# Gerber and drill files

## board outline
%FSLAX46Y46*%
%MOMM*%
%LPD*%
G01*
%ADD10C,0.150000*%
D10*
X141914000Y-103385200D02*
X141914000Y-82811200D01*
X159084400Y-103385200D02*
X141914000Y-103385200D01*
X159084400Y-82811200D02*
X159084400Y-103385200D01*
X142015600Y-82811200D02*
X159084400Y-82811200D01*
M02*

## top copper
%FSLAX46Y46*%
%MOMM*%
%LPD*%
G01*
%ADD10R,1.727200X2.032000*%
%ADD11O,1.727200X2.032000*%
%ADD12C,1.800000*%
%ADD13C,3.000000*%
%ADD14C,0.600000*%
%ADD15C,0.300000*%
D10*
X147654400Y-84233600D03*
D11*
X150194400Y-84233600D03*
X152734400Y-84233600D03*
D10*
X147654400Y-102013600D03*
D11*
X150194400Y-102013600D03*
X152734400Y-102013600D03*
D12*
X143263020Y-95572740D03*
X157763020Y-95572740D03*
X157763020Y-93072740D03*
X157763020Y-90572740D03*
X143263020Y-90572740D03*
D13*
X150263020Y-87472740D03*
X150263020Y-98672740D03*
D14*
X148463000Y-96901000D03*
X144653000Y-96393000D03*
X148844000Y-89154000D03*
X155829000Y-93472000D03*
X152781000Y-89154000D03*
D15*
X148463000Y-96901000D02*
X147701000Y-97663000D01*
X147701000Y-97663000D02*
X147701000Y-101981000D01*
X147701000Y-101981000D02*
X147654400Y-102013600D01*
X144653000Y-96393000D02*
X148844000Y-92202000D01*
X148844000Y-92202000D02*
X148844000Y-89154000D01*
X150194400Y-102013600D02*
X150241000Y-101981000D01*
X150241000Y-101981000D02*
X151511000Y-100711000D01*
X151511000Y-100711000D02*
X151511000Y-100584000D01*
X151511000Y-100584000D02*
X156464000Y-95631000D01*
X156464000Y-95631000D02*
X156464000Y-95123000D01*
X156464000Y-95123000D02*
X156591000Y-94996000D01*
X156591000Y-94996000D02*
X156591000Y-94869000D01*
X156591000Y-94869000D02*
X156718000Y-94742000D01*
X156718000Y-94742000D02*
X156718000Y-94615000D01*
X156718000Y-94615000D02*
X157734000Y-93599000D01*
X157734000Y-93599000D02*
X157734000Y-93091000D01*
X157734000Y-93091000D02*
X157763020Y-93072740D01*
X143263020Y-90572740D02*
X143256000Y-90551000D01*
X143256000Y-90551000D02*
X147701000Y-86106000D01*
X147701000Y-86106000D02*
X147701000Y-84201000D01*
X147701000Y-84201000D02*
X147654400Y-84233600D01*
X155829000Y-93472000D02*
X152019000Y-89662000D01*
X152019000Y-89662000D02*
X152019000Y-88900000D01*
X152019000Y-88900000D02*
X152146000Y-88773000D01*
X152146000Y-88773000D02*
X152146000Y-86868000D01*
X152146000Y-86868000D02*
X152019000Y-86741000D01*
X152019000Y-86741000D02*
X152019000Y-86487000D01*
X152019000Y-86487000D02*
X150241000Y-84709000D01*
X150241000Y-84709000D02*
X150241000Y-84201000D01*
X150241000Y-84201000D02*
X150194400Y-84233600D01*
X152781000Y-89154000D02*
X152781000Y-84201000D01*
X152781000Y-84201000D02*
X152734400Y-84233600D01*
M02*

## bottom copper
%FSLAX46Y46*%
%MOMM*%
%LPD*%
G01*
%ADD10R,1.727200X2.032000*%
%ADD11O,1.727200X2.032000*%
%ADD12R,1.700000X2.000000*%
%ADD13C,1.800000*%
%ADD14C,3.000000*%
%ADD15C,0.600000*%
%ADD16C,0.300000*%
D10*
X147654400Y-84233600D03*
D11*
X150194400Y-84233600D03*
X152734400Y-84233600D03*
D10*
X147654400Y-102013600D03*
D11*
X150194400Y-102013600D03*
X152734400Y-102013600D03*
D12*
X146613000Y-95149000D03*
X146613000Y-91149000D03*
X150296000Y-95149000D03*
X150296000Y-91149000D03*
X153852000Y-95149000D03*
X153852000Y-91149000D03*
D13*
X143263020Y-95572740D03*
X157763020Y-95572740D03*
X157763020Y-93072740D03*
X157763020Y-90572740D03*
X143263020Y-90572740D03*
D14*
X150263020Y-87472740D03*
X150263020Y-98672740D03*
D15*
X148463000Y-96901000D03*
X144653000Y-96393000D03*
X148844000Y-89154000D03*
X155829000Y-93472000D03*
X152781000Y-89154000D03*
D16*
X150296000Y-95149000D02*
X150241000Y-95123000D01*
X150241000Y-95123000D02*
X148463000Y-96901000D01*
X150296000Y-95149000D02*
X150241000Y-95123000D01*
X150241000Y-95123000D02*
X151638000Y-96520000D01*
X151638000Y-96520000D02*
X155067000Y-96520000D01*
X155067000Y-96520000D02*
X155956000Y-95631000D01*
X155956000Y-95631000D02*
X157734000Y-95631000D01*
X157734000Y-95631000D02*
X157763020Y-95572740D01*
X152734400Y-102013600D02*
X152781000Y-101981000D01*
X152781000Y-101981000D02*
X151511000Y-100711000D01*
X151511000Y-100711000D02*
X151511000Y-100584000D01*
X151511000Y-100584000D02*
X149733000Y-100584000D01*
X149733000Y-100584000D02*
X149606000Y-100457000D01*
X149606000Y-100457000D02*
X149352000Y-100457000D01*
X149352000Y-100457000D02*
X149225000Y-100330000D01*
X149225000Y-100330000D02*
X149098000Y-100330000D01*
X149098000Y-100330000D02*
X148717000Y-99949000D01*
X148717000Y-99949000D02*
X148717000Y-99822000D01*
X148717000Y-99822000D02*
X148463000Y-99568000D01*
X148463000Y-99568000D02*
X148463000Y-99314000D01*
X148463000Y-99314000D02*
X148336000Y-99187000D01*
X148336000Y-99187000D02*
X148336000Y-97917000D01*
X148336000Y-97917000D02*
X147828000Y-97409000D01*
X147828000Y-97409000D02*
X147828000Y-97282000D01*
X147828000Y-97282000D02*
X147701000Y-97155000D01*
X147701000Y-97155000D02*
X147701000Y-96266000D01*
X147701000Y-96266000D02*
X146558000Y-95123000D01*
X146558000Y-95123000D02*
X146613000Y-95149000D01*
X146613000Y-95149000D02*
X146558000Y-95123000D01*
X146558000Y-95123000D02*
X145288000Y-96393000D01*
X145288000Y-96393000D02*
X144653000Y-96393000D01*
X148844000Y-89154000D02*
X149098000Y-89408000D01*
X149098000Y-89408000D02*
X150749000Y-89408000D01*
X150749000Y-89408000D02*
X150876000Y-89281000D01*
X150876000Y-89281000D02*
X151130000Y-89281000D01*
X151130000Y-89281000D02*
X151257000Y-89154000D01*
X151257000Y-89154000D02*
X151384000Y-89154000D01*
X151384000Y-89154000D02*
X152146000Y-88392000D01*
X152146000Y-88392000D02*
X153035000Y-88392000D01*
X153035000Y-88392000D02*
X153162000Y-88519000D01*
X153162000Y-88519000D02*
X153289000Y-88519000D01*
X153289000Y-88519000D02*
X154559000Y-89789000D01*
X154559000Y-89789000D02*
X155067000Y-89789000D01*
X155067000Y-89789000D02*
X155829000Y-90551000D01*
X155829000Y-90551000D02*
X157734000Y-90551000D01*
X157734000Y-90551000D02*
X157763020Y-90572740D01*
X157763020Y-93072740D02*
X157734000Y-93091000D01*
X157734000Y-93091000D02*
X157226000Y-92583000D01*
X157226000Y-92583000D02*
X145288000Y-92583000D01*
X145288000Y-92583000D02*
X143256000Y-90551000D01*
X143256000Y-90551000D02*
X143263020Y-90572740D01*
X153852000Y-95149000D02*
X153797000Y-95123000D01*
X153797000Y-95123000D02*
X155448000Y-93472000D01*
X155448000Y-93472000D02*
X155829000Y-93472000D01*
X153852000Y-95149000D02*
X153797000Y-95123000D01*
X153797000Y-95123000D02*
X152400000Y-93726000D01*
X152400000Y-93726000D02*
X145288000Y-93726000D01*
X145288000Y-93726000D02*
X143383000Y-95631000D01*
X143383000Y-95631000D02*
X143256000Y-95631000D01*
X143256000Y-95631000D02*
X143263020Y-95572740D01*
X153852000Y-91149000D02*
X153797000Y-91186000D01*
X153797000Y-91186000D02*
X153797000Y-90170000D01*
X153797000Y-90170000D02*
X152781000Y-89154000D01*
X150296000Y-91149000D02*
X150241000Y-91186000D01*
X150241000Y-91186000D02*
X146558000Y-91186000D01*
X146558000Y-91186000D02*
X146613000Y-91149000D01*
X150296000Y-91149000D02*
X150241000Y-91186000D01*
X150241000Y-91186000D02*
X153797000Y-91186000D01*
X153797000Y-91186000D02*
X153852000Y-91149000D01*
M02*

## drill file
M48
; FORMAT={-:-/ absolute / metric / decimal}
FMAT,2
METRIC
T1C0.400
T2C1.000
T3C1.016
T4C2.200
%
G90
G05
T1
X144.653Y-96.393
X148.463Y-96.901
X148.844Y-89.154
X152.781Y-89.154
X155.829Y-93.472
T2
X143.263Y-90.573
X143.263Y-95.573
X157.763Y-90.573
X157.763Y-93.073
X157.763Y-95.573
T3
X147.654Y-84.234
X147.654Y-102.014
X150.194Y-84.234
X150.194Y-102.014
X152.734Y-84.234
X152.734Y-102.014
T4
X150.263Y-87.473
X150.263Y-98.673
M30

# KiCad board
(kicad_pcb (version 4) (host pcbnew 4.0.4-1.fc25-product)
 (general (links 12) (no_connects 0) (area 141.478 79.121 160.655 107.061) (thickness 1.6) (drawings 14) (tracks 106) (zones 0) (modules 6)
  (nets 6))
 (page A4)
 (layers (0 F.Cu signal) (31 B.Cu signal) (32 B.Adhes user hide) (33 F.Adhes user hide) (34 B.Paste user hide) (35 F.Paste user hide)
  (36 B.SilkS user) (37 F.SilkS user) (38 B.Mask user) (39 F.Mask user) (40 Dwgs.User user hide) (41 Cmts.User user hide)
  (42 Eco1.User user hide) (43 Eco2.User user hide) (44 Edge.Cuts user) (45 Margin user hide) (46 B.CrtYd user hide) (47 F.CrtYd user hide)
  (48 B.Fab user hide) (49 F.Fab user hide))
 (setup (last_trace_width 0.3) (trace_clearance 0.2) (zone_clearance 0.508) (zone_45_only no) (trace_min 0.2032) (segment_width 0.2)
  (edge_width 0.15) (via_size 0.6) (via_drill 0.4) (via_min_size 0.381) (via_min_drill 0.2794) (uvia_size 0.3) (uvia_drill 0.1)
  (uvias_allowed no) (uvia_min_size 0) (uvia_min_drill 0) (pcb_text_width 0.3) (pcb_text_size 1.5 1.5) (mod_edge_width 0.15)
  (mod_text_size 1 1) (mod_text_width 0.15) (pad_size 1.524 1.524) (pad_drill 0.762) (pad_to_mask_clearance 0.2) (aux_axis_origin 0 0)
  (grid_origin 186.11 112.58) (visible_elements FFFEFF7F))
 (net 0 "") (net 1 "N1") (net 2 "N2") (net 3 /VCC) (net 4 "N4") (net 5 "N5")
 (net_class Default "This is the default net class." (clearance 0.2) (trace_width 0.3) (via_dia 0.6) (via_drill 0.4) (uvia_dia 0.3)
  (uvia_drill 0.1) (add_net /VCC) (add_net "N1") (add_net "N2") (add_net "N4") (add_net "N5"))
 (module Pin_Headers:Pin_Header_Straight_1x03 (layer F.Cu) (at 147.6544 84.2336 90)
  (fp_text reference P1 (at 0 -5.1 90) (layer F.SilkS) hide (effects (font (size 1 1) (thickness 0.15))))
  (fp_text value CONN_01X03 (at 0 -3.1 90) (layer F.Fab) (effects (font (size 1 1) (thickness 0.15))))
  (pad 1 thru_hole rect (at 0 0 90) (size 2.032 1.7272) (drill 1.016) (layers *.Cu *.Mask F.SilkS) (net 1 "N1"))
  (pad 2 thru_hole oval (at 0 2.54 90) (size 2.032 1.7272) (drill 1.016) (layers *.Cu *.Mask F.SilkS) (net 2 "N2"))
  (pad 3 thru_hole oval (at 0 5.08 90) (size 2.032 1.7272) (drill 1.016) (layers *.Cu *.Mask F.SilkS) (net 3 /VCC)))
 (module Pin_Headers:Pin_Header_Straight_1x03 (layer F.Cu) (at 147.6544 102.0136 90)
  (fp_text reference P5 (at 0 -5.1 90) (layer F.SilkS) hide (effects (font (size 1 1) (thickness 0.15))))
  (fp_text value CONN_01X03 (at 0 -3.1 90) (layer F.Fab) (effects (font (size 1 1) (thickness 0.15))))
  (pad 1 thru_hole rect (at 0 0 90) (size 2.032 1.7272) (drill 1.016) (layers *.Cu *.Mask F.SilkS) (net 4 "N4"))
  (pad 2 thru_hole oval (at 0 2.54 90) (size 2.032 1.7272) (drill 1.016) (layers *.Cu *.Mask F.SilkS) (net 1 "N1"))
  (pad 3 thru_hole oval (at 0 5.08 90) (size 2.032 1.7272) (drill 1.016) (layers *.Cu *.Mask F.SilkS) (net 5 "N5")))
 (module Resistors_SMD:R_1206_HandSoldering (layer B.Cu) (at 146.613 93.149 90)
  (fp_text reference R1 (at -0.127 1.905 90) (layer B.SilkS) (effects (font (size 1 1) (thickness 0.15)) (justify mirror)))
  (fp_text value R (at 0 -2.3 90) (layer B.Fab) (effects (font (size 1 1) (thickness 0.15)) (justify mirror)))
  (pad 1 smd rect (at -2 0 90) (size 2 1.7) (layers B.Cu B.Paste B.Mask) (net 5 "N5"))
  (pad 2 smd rect (at 2 0 90) (size 2 1.7) (layers B.Cu B.Paste B.Mask) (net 3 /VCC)))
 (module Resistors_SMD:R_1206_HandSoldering (layer B.Cu) (at 150.296 93.149 90)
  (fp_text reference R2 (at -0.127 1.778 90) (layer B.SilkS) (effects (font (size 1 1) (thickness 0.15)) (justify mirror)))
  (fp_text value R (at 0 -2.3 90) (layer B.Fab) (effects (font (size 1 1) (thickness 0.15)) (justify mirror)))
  (pad 1 smd rect (at -2 0 90) (size 2 1.7) (layers B.Cu B.Paste B.Mask) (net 4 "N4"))
  (pad 2 smd rect (at 2 0 90) (size 2 1.7) (layers B.Cu B.Paste B.Mask) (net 3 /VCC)))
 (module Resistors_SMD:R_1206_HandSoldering (layer B.Cu) (at 153.852 93.149 90)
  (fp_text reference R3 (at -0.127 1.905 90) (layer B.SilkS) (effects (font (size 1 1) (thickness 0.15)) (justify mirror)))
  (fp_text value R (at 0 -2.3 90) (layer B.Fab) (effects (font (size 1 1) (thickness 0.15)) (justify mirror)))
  (pad 1 smd rect (at -2 0 90) (size 2 1.7) (layers B.Cu B.Paste B.Mask) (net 2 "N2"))
  (pad 2 smd rect (at 2 0 90) (size 2 1.7) (layers B.Cu B.Paste B.Mask) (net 3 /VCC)))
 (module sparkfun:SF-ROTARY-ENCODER (layer F.Cu) (at 150.26302 93.07274 90)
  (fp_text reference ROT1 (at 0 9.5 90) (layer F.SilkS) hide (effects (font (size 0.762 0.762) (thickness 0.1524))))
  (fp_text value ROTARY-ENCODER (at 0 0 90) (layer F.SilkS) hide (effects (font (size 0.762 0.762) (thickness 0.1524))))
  (pad 1 thru_hole circle (at -2.5 -7 90) (size 1.8 1.8) (drill 1) (layers *.Cu *.Mask F.SilkS) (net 2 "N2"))
  (pad 2 thru_hole circle (at -2.5 7.5 90) (size 1.8 1.8) (drill 1) (layers *.Cu *.Mask F.SilkS) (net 4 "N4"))
  (pad 3 thru_hole circle (at 0 7.5 90) (size 1.8 1.8) (drill 1) (layers *.Cu *.Mask F.SilkS) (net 1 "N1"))
  (pad 4 thru_hole circle (at 2.5 7.5 90) (size 1.8 1.8) (drill 1) (layers *.Cu *.Mask F.SilkS) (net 5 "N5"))
  (pad 5 thru_hole circle (at 2.5 -7 90) (size 1.8 1.8) (drill 1) (layers *.Cu *.Mask F.SilkS) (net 1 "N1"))
  (pad "" thru_hole circle (at 5.6 0 90) (size 3 3) (drill 2.2) (layers *.Cu *.Mask F.SilkS))
  (pad "" thru_hole circle (at -5.6 0 90) (size 3 3) (drill 2.2) (layers *.Cu *.Mask F.SilkS)))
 (gr_line (start 141.914 103.3852) (end 141.914 82.8112) (angle 90) (layer Edge.Cuts) (width 0.15))
 (gr_line (start 159.0844 103.3852) (end 141.914 103.3852) (angle 90) (layer Edge.Cuts) (width 0.15))
 (gr_line (start 159.0844 82.8112) (end 159.0844 103.3852) (angle 90) (layer Edge.Cuts) (width 0.15))
 (gr_line (start 142.0156 82.8112) (end 159.0844 82.8112) (angle 90) (layer Edge.Cuts) (width 0.15))
 (segment (start 150.296 95.149) (end 150.241 95.123) (width 0.3) (layer B.Cu) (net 4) (status 80000))
 (segment (start 150.241 95.123) (end 148.463 96.901) (width 0.3) (layer B.Cu) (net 4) (status 80000))
 (via (at 148.463 96.901) (size 0.6) (layers F.Cu B.Cu) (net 4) (status 80000))
 (segment (start 148.463 96.901) (end 147.701 97.663) (width 0.3) (layer F.Cu) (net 4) (status 80000))
 (segment (start 147.701 97.663) (end 147.701 101.981) (width 0.3) (layer F.Cu) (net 4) (status 80000))
 (segment (start 147.701 101.981) (end 147.6544 102.0136) (width 0.3) (layer F.Cu) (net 4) (status 80000))
 (segment (start 150.296 95.149) (end 150.241 95.123) (width 0.3) (layer B.Cu) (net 4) (status 80000))
 (segment (start 150.241 95.123) (end 151.638 96.52) (width 0.3) (layer B.Cu) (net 4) (status 80000))
 (segment (start 151.638 96.52) (end 155.067 96.52) (width 0.3) (layer B.Cu) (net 4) (status 80000))
 (segment (start 155.067 96.52) (end 155.956 95.631) (width 0.3) (layer B.Cu) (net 4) (status 80000))
 (segment (start 155.956 95.631) (end 157.734 95.631) (width 0.3) (layer B.Cu) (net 4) (status 80000))
 (segment (start 157.734 95.631) (end 157.76302 95.57274) (width 0.3) (layer B.Cu) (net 4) (status 80000))
 (segment (start 152.7344 102.0136) (end 152.781 101.981) (width 0.3) (layer B.Cu) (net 5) (status 80000))
 (segment (start 152.781 101.981) (end 151.511 100.711) (width 0.3) (layer B.Cu) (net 5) (status 80000))
 (segment (start 151.511 100.711) (end 151.511 100.584) (width 0.3) (layer B.Cu) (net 5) (status 80000))
 (segment (start 151.511 100.584) (end 149.733 100.584) (width 0.3) (layer B.Cu) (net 5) (status 80000))
 (segment (start 149.733 100.584) (end 149.606 100.457) (width 0.3) (layer B.Cu) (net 5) (status 80000))
 (segment (start 149.606 100.457) (end 149.352 100.457) (width 0.3) (layer B.Cu) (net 5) (status 80000))
 (segment (start 149.352 100.457) (end 149.225 100.33) (width 0.3) (layer B.Cu) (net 5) (status 80000))
 (segment (start 149.225 100.33) (end 149.098 100.33) (width 0.3) (layer B.Cu) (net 5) (status 80000))
 (segment (start 149.098 100.33) (end 148.717 99.949) (width 0.3) (layer B.Cu) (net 5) (status 80000))
 (segment (start 148.717 99.949) (end 148.717 99.822) (width 0.3) (layer B.Cu) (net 5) (status 80000))
 (segment (start 148.717 99.822) (end 148.463 99.568) (width 0.3) (layer B.Cu) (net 5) (status 80000))
 (segment (start 148.463 99.568) (end 148.463 99.314) (width 0.3) (layer B.Cu) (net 5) (status 80000))
 (segment (start 148.463 99.314) (end 148.336 99.187) (width 0.3) (layer B.Cu) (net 5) (status 80000))
 (segment (start 148.336 99.187) (end 148.336 97.917) (width 0.3) (layer B.Cu) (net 5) (status 80000))
 (segment (start 148.336 97.917) (end 147.828 97.409) (width 0.3) (layer B.Cu) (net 5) (status 80000))
 (segment (start 147.828 97.409) (end 147.828 97.282) (width 0.3) (layer B.Cu) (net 5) (status 80000))
 (segment (start 147.828 97.282) (end 147.701 97.155) (width 0.3) (layer B.Cu) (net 5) (status 80000))
 (segment (start 147.701 97.155) (end 147.701 96.266) (width 0.3) (layer B.Cu) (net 5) (status 80000))
 (segment (start 147.701 96.266) (end 146.558 95.123) (width 0.3) (layer B.Cu) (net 5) (status 80000))
 (segment (start 146.558 95.123) (end 146.613 95.149) (width 0.3) (layer B.Cu) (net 5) (status 80000))
 (segment (start 146.613 95.149) (end 146.558 95.123) (width 0.3) (layer B.Cu) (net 5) (status 80000))
 (segment (start 146.558 95.123) (end 145.288 96.393) (width 0.3) (layer B.Cu) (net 5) (status 80000))
 (segment (start 145.288 96.393) (end 144.653 96.393) (width 0.3) (layer B.Cu) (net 5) (status 80000))
 (via (at 144.653 96.393) (size 0.6) (layers F.Cu B.Cu) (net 5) (status 80000))
 (segment (start 144.653 96.393) (end 148.844 92.202) (width 0.3) (layer F.Cu) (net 5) (status 80000))
 (segment (start 148.844 92.202) (end 148.844 89.154) (width 0.3) (layer F.Cu) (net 5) (status 80000))
 (via (at 148.844 89.154) (size 0.6) (layers F.Cu B.Cu) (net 5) (status 80000))
 (segment (start 148.844 89.154) (end 149.098 89.408) (width 0.3) (layer B.Cu) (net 5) (status 80000))
 (segment (start 149.098 89.408) (end 150.749 89.408) (width 0.3) (layer B.Cu) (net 5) (status 80000))
 (segment (start 150.749 89.408) (end 150.876 89.281) (width 0.3) (layer B.Cu) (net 5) (status 80000))
 (segment (start 150.876 89.281) (end 151.13 89.281) (width 0.3) (layer B.Cu) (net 5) (status 80000))
 (segment (start 151.13 89.281) (end 151.257 89.154) (width 0.3) (layer B.Cu) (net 5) (status 80000))
 (segment (start 151.257 89.154) (end 151.384 89.154) (width 0.3) (layer B.Cu) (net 5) (status 80000))
 (segment (start 151.384 89.154) (end 152.146 88.392) (width 0.3) (layer B.Cu) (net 5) (status 80000))
 (segment (start 152.146 88.392) (end 153.035 88.392) (width 0.3) (layer B.Cu) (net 5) (status 80000))
 (segment (start 153.035 88.392) (end 153.162 88.519) (width 0.3) (layer B.Cu) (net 5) (status 80000))
 (segment (start 153.162 88.519) (end 153.289 88.519) (width 0.3) (layer B.Cu) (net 5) (status 80000))
 (segment (start 153.289 88.519) (end 154.559 89.789) (width 0.3) (layer B.Cu) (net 5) (status 80000))
 (segment (start 154.559 89.789) (end 155.067 89.789) (width 0.3) (layer B.Cu) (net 5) (status 80000))
 (segment (start 155.067 89.789) (end 155.829 90.551) (width 0.3) (layer B.Cu) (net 5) (status 80000))
 (segment (start 155.829 90.551) (end 157.734 90.551) (width 0.3) (layer B.Cu) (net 5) (status 80000))
 (segment (start 157.734 90.551) (end 157.76302 90.57274) (width 0.3) (layer B.Cu) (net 5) (status 80000))
 (segment (start 150.1944 102.0136) (end 150.241 101.981) (width 0.3) (layer F.Cu) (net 1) (status 80000))
 (segment (start 150.241 101.981) (end 151.511 100.711) (width 0.3) (layer F.Cu) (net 1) (status 80000))
 (segment (start 151.511 100.711) (end 151.511 100.584) (width 0.3) (layer F.Cu) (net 1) (status 80000))
 (segment (start 151.511 100.584) (end 156.464 95.631) (width 0.3) (layer F.Cu) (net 1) (status 80000))
 (segment (start 156.464 95.631) (end 156.464 95.123) (width 0.3) (layer F.Cu) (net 1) (status 80000))
 (segment (start 156.464 95.123) (end 156.591 94.996) (width 0.3) (layer F.Cu) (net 1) (status 80000))
 (segment (start 156.591 94.996) (end 156.591 94.869) (width 0.3) (layer F.Cu) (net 1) (status 80000))
 (segment (start 156.591 94.869) (end 156.718 94.742) (width 0.3) (layer F.Cu) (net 1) (status 80000))
 (segment (start 156.718 94.742) (end 156.718 94.615) (width 0.3) (layer F.Cu) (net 1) (status 80000))
 (segment (start 156.718 94.615) (end 157.734 93.599) (width 0.3) (layer F.Cu) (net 1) (status 80000))
 (segment (start 157.734 93.599) (end 157.734 93.091) (width 0.3) (layer F.Cu) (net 1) (status 80000))
 (segment (start 157.734 93.091) (end 157.76302 93.07274) (width 0.3) (layer F.Cu) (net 1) (status 80000))
 (segment (start 143.26302 90.57274) (end 143.256 90.551) (width 0.3) (layer F.Cu) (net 1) (status 80000))
 (segment (start 143.256 90.551) (end 147.701 86.106) (width 0.3) (layer F.Cu) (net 1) (status 80000))
 (segment (start 147.701 86.106) (end 147.701 84.201) (width 0.3) (layer F.Cu) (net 1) (status 80000))
 (segment (start 147.701 84.201) (end 147.6544 84.2336) (width 0.3) (layer F.Cu) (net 1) (status 80000))
 (segment (start 157.76302 93.07274) (end 157.734 93.091) (width 0.3) (layer B.Cu) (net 1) (status 80000))
 (segment (start 157.734 93.091) (end 157.226 92.583) (width 0.3) (layer B.Cu) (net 1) (status 80000))
 (segment (start 157.226 92.583) (end 145.288 92.583) (width 0.3) (layer B.Cu) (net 1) (status 80000))
 (segment (start 145.288 92.583) (end 143.256 90.551) (width 0.3) (layer B.Cu) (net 1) (status 80000))
 (segment (start 143.256 90.551) (end 143.26302 90.57274) (width 0.3) (layer B.Cu) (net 1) (status 80000))
 (segment (start 153.852 95.149) (end 153.797 95.123) (width 0.3) (layer B.Cu) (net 2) (status 80000))
 (segment (start 153.797 95.123) (end 155.448 93.472) (width 0.3) (layer B.Cu) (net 2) (status 80000))
 (segment (start 155.448 93.472) (end 155.829 93.472) (width 0.3) (layer B.Cu) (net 2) (status 80000))
 (via (at 155.829 93.472) (size 0.6) (layers F.Cu B.Cu) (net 2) (status 80000))
 (segment (start 155.829 93.472) (end 152.019 89.662) (width 0.3) (layer F.Cu) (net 2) (status 80000))
 (segment (start 152.019 89.662) (end 152.019 88.9) (width 0.3) (layer F.Cu) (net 2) (status 80000))
 (segment (start 152.019 88.9) (end 152.146 88.773) (width 0.3) (layer F.Cu) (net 2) (status 80000))
 (segment (start 152.146 88.773) (end 152.146 86.868) (width 0.3) (layer F.Cu) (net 2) (status 80000))
 (segment (start 152.146 86.868) (end 152.019 86.741) (width 0.3) (layer F.Cu) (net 2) (status 80000))
 (segment (start 152.019 86.741) (end 152.019 86.487) (width 0.3) (layer F.Cu) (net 2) (status 80000))
 (segment (start 152.019 86.487) (end 150.241 84.709) (width 0.3) (layer F.Cu) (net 2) (status 80000))
 (segment (start 150.241 84.709) (end 150.241 84.201) (width 0.3) (layer F.Cu) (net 2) (status 80000))
 (segment (start 150.241 84.201) (end 150.1944 84.2336) (width 0.3) (layer F.Cu) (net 2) (status 80000))
 (segment (start 153.852 95.149) (end 153.797 95.123) (width 0.3) (layer B.Cu) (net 2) (status 80000))
 (segment (start 153.797 95.123) (end 152.4 93.726) (width 0.3) (layer B.Cu) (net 2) (status 80000))
 (segment (start 152.4 93.726) (end 145.288 93.726) (width 0.3) (layer B.Cu) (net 2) (status 80000))
 (segment (start 145.288 93.726) (end 143.383 95.631) (width 0.3) (layer B.Cu) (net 2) (status 80000))
 (segment (start 143.383 95.631) (end 143.256 95.631) (width 0.3) (layer B.Cu) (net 2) (status 80000))
 (segment (start 143.256 95.631) (end 143.26302 95.57274) (width 0.3) (layer B.Cu) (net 2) (status 80000))
 (segment (start 153.852 91.149) (end 153.797 91.186) (width 0.3) (layer B.Cu) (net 3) (status 80000))
 (segment (start 153.797 91.186) (end 153.797 90.17) (width 0.3) (layer B.Cu) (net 3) (status 80000))
 (segment (start 153.797 90.17) (end 152.781 89.154) (width 0.3) (layer B.Cu) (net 3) (status 80000))
 (via (at 152.781 89.154) (size 0.6) (layers F.Cu B.Cu) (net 3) (status 80000))
 (segment (start 152.781 89.154) (end 152.781 84.201) (width 0.3) (layer F.Cu) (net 3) (status 80000))
 (segment (start 152.781 84.201) (end 152.7344 84.2336) (width 0.3) (layer F.Cu) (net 3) (status 80000))
 (segment (start 150.296 91.149) (end 150.241 91.186) (width 0.3) (layer B.Cu) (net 3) (status 80000))
 (segment (start 150.241 91.186) (end 146.558 91.186) (width 0.3) (layer B.Cu) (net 3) (status 80000))
 (segment (start 146.558 91.186) (end 146.613 91.149) (width 0.3) (layer B.Cu) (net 3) (status 80000))
 (segment (start 150.296 91.149) (end 150.241 91.186) (width 0.3) (layer B.Cu) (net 3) (status 80000))
 (segment (start 150.241 91.186) (end 153.797 91.186) (width 0.3) (layer B.Cu) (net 3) (status 80000))
 (segment (start 153.797 91.186) (end 153.852 91.149) (width 0.3) (layer B.Cu) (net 3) (status 80000)))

